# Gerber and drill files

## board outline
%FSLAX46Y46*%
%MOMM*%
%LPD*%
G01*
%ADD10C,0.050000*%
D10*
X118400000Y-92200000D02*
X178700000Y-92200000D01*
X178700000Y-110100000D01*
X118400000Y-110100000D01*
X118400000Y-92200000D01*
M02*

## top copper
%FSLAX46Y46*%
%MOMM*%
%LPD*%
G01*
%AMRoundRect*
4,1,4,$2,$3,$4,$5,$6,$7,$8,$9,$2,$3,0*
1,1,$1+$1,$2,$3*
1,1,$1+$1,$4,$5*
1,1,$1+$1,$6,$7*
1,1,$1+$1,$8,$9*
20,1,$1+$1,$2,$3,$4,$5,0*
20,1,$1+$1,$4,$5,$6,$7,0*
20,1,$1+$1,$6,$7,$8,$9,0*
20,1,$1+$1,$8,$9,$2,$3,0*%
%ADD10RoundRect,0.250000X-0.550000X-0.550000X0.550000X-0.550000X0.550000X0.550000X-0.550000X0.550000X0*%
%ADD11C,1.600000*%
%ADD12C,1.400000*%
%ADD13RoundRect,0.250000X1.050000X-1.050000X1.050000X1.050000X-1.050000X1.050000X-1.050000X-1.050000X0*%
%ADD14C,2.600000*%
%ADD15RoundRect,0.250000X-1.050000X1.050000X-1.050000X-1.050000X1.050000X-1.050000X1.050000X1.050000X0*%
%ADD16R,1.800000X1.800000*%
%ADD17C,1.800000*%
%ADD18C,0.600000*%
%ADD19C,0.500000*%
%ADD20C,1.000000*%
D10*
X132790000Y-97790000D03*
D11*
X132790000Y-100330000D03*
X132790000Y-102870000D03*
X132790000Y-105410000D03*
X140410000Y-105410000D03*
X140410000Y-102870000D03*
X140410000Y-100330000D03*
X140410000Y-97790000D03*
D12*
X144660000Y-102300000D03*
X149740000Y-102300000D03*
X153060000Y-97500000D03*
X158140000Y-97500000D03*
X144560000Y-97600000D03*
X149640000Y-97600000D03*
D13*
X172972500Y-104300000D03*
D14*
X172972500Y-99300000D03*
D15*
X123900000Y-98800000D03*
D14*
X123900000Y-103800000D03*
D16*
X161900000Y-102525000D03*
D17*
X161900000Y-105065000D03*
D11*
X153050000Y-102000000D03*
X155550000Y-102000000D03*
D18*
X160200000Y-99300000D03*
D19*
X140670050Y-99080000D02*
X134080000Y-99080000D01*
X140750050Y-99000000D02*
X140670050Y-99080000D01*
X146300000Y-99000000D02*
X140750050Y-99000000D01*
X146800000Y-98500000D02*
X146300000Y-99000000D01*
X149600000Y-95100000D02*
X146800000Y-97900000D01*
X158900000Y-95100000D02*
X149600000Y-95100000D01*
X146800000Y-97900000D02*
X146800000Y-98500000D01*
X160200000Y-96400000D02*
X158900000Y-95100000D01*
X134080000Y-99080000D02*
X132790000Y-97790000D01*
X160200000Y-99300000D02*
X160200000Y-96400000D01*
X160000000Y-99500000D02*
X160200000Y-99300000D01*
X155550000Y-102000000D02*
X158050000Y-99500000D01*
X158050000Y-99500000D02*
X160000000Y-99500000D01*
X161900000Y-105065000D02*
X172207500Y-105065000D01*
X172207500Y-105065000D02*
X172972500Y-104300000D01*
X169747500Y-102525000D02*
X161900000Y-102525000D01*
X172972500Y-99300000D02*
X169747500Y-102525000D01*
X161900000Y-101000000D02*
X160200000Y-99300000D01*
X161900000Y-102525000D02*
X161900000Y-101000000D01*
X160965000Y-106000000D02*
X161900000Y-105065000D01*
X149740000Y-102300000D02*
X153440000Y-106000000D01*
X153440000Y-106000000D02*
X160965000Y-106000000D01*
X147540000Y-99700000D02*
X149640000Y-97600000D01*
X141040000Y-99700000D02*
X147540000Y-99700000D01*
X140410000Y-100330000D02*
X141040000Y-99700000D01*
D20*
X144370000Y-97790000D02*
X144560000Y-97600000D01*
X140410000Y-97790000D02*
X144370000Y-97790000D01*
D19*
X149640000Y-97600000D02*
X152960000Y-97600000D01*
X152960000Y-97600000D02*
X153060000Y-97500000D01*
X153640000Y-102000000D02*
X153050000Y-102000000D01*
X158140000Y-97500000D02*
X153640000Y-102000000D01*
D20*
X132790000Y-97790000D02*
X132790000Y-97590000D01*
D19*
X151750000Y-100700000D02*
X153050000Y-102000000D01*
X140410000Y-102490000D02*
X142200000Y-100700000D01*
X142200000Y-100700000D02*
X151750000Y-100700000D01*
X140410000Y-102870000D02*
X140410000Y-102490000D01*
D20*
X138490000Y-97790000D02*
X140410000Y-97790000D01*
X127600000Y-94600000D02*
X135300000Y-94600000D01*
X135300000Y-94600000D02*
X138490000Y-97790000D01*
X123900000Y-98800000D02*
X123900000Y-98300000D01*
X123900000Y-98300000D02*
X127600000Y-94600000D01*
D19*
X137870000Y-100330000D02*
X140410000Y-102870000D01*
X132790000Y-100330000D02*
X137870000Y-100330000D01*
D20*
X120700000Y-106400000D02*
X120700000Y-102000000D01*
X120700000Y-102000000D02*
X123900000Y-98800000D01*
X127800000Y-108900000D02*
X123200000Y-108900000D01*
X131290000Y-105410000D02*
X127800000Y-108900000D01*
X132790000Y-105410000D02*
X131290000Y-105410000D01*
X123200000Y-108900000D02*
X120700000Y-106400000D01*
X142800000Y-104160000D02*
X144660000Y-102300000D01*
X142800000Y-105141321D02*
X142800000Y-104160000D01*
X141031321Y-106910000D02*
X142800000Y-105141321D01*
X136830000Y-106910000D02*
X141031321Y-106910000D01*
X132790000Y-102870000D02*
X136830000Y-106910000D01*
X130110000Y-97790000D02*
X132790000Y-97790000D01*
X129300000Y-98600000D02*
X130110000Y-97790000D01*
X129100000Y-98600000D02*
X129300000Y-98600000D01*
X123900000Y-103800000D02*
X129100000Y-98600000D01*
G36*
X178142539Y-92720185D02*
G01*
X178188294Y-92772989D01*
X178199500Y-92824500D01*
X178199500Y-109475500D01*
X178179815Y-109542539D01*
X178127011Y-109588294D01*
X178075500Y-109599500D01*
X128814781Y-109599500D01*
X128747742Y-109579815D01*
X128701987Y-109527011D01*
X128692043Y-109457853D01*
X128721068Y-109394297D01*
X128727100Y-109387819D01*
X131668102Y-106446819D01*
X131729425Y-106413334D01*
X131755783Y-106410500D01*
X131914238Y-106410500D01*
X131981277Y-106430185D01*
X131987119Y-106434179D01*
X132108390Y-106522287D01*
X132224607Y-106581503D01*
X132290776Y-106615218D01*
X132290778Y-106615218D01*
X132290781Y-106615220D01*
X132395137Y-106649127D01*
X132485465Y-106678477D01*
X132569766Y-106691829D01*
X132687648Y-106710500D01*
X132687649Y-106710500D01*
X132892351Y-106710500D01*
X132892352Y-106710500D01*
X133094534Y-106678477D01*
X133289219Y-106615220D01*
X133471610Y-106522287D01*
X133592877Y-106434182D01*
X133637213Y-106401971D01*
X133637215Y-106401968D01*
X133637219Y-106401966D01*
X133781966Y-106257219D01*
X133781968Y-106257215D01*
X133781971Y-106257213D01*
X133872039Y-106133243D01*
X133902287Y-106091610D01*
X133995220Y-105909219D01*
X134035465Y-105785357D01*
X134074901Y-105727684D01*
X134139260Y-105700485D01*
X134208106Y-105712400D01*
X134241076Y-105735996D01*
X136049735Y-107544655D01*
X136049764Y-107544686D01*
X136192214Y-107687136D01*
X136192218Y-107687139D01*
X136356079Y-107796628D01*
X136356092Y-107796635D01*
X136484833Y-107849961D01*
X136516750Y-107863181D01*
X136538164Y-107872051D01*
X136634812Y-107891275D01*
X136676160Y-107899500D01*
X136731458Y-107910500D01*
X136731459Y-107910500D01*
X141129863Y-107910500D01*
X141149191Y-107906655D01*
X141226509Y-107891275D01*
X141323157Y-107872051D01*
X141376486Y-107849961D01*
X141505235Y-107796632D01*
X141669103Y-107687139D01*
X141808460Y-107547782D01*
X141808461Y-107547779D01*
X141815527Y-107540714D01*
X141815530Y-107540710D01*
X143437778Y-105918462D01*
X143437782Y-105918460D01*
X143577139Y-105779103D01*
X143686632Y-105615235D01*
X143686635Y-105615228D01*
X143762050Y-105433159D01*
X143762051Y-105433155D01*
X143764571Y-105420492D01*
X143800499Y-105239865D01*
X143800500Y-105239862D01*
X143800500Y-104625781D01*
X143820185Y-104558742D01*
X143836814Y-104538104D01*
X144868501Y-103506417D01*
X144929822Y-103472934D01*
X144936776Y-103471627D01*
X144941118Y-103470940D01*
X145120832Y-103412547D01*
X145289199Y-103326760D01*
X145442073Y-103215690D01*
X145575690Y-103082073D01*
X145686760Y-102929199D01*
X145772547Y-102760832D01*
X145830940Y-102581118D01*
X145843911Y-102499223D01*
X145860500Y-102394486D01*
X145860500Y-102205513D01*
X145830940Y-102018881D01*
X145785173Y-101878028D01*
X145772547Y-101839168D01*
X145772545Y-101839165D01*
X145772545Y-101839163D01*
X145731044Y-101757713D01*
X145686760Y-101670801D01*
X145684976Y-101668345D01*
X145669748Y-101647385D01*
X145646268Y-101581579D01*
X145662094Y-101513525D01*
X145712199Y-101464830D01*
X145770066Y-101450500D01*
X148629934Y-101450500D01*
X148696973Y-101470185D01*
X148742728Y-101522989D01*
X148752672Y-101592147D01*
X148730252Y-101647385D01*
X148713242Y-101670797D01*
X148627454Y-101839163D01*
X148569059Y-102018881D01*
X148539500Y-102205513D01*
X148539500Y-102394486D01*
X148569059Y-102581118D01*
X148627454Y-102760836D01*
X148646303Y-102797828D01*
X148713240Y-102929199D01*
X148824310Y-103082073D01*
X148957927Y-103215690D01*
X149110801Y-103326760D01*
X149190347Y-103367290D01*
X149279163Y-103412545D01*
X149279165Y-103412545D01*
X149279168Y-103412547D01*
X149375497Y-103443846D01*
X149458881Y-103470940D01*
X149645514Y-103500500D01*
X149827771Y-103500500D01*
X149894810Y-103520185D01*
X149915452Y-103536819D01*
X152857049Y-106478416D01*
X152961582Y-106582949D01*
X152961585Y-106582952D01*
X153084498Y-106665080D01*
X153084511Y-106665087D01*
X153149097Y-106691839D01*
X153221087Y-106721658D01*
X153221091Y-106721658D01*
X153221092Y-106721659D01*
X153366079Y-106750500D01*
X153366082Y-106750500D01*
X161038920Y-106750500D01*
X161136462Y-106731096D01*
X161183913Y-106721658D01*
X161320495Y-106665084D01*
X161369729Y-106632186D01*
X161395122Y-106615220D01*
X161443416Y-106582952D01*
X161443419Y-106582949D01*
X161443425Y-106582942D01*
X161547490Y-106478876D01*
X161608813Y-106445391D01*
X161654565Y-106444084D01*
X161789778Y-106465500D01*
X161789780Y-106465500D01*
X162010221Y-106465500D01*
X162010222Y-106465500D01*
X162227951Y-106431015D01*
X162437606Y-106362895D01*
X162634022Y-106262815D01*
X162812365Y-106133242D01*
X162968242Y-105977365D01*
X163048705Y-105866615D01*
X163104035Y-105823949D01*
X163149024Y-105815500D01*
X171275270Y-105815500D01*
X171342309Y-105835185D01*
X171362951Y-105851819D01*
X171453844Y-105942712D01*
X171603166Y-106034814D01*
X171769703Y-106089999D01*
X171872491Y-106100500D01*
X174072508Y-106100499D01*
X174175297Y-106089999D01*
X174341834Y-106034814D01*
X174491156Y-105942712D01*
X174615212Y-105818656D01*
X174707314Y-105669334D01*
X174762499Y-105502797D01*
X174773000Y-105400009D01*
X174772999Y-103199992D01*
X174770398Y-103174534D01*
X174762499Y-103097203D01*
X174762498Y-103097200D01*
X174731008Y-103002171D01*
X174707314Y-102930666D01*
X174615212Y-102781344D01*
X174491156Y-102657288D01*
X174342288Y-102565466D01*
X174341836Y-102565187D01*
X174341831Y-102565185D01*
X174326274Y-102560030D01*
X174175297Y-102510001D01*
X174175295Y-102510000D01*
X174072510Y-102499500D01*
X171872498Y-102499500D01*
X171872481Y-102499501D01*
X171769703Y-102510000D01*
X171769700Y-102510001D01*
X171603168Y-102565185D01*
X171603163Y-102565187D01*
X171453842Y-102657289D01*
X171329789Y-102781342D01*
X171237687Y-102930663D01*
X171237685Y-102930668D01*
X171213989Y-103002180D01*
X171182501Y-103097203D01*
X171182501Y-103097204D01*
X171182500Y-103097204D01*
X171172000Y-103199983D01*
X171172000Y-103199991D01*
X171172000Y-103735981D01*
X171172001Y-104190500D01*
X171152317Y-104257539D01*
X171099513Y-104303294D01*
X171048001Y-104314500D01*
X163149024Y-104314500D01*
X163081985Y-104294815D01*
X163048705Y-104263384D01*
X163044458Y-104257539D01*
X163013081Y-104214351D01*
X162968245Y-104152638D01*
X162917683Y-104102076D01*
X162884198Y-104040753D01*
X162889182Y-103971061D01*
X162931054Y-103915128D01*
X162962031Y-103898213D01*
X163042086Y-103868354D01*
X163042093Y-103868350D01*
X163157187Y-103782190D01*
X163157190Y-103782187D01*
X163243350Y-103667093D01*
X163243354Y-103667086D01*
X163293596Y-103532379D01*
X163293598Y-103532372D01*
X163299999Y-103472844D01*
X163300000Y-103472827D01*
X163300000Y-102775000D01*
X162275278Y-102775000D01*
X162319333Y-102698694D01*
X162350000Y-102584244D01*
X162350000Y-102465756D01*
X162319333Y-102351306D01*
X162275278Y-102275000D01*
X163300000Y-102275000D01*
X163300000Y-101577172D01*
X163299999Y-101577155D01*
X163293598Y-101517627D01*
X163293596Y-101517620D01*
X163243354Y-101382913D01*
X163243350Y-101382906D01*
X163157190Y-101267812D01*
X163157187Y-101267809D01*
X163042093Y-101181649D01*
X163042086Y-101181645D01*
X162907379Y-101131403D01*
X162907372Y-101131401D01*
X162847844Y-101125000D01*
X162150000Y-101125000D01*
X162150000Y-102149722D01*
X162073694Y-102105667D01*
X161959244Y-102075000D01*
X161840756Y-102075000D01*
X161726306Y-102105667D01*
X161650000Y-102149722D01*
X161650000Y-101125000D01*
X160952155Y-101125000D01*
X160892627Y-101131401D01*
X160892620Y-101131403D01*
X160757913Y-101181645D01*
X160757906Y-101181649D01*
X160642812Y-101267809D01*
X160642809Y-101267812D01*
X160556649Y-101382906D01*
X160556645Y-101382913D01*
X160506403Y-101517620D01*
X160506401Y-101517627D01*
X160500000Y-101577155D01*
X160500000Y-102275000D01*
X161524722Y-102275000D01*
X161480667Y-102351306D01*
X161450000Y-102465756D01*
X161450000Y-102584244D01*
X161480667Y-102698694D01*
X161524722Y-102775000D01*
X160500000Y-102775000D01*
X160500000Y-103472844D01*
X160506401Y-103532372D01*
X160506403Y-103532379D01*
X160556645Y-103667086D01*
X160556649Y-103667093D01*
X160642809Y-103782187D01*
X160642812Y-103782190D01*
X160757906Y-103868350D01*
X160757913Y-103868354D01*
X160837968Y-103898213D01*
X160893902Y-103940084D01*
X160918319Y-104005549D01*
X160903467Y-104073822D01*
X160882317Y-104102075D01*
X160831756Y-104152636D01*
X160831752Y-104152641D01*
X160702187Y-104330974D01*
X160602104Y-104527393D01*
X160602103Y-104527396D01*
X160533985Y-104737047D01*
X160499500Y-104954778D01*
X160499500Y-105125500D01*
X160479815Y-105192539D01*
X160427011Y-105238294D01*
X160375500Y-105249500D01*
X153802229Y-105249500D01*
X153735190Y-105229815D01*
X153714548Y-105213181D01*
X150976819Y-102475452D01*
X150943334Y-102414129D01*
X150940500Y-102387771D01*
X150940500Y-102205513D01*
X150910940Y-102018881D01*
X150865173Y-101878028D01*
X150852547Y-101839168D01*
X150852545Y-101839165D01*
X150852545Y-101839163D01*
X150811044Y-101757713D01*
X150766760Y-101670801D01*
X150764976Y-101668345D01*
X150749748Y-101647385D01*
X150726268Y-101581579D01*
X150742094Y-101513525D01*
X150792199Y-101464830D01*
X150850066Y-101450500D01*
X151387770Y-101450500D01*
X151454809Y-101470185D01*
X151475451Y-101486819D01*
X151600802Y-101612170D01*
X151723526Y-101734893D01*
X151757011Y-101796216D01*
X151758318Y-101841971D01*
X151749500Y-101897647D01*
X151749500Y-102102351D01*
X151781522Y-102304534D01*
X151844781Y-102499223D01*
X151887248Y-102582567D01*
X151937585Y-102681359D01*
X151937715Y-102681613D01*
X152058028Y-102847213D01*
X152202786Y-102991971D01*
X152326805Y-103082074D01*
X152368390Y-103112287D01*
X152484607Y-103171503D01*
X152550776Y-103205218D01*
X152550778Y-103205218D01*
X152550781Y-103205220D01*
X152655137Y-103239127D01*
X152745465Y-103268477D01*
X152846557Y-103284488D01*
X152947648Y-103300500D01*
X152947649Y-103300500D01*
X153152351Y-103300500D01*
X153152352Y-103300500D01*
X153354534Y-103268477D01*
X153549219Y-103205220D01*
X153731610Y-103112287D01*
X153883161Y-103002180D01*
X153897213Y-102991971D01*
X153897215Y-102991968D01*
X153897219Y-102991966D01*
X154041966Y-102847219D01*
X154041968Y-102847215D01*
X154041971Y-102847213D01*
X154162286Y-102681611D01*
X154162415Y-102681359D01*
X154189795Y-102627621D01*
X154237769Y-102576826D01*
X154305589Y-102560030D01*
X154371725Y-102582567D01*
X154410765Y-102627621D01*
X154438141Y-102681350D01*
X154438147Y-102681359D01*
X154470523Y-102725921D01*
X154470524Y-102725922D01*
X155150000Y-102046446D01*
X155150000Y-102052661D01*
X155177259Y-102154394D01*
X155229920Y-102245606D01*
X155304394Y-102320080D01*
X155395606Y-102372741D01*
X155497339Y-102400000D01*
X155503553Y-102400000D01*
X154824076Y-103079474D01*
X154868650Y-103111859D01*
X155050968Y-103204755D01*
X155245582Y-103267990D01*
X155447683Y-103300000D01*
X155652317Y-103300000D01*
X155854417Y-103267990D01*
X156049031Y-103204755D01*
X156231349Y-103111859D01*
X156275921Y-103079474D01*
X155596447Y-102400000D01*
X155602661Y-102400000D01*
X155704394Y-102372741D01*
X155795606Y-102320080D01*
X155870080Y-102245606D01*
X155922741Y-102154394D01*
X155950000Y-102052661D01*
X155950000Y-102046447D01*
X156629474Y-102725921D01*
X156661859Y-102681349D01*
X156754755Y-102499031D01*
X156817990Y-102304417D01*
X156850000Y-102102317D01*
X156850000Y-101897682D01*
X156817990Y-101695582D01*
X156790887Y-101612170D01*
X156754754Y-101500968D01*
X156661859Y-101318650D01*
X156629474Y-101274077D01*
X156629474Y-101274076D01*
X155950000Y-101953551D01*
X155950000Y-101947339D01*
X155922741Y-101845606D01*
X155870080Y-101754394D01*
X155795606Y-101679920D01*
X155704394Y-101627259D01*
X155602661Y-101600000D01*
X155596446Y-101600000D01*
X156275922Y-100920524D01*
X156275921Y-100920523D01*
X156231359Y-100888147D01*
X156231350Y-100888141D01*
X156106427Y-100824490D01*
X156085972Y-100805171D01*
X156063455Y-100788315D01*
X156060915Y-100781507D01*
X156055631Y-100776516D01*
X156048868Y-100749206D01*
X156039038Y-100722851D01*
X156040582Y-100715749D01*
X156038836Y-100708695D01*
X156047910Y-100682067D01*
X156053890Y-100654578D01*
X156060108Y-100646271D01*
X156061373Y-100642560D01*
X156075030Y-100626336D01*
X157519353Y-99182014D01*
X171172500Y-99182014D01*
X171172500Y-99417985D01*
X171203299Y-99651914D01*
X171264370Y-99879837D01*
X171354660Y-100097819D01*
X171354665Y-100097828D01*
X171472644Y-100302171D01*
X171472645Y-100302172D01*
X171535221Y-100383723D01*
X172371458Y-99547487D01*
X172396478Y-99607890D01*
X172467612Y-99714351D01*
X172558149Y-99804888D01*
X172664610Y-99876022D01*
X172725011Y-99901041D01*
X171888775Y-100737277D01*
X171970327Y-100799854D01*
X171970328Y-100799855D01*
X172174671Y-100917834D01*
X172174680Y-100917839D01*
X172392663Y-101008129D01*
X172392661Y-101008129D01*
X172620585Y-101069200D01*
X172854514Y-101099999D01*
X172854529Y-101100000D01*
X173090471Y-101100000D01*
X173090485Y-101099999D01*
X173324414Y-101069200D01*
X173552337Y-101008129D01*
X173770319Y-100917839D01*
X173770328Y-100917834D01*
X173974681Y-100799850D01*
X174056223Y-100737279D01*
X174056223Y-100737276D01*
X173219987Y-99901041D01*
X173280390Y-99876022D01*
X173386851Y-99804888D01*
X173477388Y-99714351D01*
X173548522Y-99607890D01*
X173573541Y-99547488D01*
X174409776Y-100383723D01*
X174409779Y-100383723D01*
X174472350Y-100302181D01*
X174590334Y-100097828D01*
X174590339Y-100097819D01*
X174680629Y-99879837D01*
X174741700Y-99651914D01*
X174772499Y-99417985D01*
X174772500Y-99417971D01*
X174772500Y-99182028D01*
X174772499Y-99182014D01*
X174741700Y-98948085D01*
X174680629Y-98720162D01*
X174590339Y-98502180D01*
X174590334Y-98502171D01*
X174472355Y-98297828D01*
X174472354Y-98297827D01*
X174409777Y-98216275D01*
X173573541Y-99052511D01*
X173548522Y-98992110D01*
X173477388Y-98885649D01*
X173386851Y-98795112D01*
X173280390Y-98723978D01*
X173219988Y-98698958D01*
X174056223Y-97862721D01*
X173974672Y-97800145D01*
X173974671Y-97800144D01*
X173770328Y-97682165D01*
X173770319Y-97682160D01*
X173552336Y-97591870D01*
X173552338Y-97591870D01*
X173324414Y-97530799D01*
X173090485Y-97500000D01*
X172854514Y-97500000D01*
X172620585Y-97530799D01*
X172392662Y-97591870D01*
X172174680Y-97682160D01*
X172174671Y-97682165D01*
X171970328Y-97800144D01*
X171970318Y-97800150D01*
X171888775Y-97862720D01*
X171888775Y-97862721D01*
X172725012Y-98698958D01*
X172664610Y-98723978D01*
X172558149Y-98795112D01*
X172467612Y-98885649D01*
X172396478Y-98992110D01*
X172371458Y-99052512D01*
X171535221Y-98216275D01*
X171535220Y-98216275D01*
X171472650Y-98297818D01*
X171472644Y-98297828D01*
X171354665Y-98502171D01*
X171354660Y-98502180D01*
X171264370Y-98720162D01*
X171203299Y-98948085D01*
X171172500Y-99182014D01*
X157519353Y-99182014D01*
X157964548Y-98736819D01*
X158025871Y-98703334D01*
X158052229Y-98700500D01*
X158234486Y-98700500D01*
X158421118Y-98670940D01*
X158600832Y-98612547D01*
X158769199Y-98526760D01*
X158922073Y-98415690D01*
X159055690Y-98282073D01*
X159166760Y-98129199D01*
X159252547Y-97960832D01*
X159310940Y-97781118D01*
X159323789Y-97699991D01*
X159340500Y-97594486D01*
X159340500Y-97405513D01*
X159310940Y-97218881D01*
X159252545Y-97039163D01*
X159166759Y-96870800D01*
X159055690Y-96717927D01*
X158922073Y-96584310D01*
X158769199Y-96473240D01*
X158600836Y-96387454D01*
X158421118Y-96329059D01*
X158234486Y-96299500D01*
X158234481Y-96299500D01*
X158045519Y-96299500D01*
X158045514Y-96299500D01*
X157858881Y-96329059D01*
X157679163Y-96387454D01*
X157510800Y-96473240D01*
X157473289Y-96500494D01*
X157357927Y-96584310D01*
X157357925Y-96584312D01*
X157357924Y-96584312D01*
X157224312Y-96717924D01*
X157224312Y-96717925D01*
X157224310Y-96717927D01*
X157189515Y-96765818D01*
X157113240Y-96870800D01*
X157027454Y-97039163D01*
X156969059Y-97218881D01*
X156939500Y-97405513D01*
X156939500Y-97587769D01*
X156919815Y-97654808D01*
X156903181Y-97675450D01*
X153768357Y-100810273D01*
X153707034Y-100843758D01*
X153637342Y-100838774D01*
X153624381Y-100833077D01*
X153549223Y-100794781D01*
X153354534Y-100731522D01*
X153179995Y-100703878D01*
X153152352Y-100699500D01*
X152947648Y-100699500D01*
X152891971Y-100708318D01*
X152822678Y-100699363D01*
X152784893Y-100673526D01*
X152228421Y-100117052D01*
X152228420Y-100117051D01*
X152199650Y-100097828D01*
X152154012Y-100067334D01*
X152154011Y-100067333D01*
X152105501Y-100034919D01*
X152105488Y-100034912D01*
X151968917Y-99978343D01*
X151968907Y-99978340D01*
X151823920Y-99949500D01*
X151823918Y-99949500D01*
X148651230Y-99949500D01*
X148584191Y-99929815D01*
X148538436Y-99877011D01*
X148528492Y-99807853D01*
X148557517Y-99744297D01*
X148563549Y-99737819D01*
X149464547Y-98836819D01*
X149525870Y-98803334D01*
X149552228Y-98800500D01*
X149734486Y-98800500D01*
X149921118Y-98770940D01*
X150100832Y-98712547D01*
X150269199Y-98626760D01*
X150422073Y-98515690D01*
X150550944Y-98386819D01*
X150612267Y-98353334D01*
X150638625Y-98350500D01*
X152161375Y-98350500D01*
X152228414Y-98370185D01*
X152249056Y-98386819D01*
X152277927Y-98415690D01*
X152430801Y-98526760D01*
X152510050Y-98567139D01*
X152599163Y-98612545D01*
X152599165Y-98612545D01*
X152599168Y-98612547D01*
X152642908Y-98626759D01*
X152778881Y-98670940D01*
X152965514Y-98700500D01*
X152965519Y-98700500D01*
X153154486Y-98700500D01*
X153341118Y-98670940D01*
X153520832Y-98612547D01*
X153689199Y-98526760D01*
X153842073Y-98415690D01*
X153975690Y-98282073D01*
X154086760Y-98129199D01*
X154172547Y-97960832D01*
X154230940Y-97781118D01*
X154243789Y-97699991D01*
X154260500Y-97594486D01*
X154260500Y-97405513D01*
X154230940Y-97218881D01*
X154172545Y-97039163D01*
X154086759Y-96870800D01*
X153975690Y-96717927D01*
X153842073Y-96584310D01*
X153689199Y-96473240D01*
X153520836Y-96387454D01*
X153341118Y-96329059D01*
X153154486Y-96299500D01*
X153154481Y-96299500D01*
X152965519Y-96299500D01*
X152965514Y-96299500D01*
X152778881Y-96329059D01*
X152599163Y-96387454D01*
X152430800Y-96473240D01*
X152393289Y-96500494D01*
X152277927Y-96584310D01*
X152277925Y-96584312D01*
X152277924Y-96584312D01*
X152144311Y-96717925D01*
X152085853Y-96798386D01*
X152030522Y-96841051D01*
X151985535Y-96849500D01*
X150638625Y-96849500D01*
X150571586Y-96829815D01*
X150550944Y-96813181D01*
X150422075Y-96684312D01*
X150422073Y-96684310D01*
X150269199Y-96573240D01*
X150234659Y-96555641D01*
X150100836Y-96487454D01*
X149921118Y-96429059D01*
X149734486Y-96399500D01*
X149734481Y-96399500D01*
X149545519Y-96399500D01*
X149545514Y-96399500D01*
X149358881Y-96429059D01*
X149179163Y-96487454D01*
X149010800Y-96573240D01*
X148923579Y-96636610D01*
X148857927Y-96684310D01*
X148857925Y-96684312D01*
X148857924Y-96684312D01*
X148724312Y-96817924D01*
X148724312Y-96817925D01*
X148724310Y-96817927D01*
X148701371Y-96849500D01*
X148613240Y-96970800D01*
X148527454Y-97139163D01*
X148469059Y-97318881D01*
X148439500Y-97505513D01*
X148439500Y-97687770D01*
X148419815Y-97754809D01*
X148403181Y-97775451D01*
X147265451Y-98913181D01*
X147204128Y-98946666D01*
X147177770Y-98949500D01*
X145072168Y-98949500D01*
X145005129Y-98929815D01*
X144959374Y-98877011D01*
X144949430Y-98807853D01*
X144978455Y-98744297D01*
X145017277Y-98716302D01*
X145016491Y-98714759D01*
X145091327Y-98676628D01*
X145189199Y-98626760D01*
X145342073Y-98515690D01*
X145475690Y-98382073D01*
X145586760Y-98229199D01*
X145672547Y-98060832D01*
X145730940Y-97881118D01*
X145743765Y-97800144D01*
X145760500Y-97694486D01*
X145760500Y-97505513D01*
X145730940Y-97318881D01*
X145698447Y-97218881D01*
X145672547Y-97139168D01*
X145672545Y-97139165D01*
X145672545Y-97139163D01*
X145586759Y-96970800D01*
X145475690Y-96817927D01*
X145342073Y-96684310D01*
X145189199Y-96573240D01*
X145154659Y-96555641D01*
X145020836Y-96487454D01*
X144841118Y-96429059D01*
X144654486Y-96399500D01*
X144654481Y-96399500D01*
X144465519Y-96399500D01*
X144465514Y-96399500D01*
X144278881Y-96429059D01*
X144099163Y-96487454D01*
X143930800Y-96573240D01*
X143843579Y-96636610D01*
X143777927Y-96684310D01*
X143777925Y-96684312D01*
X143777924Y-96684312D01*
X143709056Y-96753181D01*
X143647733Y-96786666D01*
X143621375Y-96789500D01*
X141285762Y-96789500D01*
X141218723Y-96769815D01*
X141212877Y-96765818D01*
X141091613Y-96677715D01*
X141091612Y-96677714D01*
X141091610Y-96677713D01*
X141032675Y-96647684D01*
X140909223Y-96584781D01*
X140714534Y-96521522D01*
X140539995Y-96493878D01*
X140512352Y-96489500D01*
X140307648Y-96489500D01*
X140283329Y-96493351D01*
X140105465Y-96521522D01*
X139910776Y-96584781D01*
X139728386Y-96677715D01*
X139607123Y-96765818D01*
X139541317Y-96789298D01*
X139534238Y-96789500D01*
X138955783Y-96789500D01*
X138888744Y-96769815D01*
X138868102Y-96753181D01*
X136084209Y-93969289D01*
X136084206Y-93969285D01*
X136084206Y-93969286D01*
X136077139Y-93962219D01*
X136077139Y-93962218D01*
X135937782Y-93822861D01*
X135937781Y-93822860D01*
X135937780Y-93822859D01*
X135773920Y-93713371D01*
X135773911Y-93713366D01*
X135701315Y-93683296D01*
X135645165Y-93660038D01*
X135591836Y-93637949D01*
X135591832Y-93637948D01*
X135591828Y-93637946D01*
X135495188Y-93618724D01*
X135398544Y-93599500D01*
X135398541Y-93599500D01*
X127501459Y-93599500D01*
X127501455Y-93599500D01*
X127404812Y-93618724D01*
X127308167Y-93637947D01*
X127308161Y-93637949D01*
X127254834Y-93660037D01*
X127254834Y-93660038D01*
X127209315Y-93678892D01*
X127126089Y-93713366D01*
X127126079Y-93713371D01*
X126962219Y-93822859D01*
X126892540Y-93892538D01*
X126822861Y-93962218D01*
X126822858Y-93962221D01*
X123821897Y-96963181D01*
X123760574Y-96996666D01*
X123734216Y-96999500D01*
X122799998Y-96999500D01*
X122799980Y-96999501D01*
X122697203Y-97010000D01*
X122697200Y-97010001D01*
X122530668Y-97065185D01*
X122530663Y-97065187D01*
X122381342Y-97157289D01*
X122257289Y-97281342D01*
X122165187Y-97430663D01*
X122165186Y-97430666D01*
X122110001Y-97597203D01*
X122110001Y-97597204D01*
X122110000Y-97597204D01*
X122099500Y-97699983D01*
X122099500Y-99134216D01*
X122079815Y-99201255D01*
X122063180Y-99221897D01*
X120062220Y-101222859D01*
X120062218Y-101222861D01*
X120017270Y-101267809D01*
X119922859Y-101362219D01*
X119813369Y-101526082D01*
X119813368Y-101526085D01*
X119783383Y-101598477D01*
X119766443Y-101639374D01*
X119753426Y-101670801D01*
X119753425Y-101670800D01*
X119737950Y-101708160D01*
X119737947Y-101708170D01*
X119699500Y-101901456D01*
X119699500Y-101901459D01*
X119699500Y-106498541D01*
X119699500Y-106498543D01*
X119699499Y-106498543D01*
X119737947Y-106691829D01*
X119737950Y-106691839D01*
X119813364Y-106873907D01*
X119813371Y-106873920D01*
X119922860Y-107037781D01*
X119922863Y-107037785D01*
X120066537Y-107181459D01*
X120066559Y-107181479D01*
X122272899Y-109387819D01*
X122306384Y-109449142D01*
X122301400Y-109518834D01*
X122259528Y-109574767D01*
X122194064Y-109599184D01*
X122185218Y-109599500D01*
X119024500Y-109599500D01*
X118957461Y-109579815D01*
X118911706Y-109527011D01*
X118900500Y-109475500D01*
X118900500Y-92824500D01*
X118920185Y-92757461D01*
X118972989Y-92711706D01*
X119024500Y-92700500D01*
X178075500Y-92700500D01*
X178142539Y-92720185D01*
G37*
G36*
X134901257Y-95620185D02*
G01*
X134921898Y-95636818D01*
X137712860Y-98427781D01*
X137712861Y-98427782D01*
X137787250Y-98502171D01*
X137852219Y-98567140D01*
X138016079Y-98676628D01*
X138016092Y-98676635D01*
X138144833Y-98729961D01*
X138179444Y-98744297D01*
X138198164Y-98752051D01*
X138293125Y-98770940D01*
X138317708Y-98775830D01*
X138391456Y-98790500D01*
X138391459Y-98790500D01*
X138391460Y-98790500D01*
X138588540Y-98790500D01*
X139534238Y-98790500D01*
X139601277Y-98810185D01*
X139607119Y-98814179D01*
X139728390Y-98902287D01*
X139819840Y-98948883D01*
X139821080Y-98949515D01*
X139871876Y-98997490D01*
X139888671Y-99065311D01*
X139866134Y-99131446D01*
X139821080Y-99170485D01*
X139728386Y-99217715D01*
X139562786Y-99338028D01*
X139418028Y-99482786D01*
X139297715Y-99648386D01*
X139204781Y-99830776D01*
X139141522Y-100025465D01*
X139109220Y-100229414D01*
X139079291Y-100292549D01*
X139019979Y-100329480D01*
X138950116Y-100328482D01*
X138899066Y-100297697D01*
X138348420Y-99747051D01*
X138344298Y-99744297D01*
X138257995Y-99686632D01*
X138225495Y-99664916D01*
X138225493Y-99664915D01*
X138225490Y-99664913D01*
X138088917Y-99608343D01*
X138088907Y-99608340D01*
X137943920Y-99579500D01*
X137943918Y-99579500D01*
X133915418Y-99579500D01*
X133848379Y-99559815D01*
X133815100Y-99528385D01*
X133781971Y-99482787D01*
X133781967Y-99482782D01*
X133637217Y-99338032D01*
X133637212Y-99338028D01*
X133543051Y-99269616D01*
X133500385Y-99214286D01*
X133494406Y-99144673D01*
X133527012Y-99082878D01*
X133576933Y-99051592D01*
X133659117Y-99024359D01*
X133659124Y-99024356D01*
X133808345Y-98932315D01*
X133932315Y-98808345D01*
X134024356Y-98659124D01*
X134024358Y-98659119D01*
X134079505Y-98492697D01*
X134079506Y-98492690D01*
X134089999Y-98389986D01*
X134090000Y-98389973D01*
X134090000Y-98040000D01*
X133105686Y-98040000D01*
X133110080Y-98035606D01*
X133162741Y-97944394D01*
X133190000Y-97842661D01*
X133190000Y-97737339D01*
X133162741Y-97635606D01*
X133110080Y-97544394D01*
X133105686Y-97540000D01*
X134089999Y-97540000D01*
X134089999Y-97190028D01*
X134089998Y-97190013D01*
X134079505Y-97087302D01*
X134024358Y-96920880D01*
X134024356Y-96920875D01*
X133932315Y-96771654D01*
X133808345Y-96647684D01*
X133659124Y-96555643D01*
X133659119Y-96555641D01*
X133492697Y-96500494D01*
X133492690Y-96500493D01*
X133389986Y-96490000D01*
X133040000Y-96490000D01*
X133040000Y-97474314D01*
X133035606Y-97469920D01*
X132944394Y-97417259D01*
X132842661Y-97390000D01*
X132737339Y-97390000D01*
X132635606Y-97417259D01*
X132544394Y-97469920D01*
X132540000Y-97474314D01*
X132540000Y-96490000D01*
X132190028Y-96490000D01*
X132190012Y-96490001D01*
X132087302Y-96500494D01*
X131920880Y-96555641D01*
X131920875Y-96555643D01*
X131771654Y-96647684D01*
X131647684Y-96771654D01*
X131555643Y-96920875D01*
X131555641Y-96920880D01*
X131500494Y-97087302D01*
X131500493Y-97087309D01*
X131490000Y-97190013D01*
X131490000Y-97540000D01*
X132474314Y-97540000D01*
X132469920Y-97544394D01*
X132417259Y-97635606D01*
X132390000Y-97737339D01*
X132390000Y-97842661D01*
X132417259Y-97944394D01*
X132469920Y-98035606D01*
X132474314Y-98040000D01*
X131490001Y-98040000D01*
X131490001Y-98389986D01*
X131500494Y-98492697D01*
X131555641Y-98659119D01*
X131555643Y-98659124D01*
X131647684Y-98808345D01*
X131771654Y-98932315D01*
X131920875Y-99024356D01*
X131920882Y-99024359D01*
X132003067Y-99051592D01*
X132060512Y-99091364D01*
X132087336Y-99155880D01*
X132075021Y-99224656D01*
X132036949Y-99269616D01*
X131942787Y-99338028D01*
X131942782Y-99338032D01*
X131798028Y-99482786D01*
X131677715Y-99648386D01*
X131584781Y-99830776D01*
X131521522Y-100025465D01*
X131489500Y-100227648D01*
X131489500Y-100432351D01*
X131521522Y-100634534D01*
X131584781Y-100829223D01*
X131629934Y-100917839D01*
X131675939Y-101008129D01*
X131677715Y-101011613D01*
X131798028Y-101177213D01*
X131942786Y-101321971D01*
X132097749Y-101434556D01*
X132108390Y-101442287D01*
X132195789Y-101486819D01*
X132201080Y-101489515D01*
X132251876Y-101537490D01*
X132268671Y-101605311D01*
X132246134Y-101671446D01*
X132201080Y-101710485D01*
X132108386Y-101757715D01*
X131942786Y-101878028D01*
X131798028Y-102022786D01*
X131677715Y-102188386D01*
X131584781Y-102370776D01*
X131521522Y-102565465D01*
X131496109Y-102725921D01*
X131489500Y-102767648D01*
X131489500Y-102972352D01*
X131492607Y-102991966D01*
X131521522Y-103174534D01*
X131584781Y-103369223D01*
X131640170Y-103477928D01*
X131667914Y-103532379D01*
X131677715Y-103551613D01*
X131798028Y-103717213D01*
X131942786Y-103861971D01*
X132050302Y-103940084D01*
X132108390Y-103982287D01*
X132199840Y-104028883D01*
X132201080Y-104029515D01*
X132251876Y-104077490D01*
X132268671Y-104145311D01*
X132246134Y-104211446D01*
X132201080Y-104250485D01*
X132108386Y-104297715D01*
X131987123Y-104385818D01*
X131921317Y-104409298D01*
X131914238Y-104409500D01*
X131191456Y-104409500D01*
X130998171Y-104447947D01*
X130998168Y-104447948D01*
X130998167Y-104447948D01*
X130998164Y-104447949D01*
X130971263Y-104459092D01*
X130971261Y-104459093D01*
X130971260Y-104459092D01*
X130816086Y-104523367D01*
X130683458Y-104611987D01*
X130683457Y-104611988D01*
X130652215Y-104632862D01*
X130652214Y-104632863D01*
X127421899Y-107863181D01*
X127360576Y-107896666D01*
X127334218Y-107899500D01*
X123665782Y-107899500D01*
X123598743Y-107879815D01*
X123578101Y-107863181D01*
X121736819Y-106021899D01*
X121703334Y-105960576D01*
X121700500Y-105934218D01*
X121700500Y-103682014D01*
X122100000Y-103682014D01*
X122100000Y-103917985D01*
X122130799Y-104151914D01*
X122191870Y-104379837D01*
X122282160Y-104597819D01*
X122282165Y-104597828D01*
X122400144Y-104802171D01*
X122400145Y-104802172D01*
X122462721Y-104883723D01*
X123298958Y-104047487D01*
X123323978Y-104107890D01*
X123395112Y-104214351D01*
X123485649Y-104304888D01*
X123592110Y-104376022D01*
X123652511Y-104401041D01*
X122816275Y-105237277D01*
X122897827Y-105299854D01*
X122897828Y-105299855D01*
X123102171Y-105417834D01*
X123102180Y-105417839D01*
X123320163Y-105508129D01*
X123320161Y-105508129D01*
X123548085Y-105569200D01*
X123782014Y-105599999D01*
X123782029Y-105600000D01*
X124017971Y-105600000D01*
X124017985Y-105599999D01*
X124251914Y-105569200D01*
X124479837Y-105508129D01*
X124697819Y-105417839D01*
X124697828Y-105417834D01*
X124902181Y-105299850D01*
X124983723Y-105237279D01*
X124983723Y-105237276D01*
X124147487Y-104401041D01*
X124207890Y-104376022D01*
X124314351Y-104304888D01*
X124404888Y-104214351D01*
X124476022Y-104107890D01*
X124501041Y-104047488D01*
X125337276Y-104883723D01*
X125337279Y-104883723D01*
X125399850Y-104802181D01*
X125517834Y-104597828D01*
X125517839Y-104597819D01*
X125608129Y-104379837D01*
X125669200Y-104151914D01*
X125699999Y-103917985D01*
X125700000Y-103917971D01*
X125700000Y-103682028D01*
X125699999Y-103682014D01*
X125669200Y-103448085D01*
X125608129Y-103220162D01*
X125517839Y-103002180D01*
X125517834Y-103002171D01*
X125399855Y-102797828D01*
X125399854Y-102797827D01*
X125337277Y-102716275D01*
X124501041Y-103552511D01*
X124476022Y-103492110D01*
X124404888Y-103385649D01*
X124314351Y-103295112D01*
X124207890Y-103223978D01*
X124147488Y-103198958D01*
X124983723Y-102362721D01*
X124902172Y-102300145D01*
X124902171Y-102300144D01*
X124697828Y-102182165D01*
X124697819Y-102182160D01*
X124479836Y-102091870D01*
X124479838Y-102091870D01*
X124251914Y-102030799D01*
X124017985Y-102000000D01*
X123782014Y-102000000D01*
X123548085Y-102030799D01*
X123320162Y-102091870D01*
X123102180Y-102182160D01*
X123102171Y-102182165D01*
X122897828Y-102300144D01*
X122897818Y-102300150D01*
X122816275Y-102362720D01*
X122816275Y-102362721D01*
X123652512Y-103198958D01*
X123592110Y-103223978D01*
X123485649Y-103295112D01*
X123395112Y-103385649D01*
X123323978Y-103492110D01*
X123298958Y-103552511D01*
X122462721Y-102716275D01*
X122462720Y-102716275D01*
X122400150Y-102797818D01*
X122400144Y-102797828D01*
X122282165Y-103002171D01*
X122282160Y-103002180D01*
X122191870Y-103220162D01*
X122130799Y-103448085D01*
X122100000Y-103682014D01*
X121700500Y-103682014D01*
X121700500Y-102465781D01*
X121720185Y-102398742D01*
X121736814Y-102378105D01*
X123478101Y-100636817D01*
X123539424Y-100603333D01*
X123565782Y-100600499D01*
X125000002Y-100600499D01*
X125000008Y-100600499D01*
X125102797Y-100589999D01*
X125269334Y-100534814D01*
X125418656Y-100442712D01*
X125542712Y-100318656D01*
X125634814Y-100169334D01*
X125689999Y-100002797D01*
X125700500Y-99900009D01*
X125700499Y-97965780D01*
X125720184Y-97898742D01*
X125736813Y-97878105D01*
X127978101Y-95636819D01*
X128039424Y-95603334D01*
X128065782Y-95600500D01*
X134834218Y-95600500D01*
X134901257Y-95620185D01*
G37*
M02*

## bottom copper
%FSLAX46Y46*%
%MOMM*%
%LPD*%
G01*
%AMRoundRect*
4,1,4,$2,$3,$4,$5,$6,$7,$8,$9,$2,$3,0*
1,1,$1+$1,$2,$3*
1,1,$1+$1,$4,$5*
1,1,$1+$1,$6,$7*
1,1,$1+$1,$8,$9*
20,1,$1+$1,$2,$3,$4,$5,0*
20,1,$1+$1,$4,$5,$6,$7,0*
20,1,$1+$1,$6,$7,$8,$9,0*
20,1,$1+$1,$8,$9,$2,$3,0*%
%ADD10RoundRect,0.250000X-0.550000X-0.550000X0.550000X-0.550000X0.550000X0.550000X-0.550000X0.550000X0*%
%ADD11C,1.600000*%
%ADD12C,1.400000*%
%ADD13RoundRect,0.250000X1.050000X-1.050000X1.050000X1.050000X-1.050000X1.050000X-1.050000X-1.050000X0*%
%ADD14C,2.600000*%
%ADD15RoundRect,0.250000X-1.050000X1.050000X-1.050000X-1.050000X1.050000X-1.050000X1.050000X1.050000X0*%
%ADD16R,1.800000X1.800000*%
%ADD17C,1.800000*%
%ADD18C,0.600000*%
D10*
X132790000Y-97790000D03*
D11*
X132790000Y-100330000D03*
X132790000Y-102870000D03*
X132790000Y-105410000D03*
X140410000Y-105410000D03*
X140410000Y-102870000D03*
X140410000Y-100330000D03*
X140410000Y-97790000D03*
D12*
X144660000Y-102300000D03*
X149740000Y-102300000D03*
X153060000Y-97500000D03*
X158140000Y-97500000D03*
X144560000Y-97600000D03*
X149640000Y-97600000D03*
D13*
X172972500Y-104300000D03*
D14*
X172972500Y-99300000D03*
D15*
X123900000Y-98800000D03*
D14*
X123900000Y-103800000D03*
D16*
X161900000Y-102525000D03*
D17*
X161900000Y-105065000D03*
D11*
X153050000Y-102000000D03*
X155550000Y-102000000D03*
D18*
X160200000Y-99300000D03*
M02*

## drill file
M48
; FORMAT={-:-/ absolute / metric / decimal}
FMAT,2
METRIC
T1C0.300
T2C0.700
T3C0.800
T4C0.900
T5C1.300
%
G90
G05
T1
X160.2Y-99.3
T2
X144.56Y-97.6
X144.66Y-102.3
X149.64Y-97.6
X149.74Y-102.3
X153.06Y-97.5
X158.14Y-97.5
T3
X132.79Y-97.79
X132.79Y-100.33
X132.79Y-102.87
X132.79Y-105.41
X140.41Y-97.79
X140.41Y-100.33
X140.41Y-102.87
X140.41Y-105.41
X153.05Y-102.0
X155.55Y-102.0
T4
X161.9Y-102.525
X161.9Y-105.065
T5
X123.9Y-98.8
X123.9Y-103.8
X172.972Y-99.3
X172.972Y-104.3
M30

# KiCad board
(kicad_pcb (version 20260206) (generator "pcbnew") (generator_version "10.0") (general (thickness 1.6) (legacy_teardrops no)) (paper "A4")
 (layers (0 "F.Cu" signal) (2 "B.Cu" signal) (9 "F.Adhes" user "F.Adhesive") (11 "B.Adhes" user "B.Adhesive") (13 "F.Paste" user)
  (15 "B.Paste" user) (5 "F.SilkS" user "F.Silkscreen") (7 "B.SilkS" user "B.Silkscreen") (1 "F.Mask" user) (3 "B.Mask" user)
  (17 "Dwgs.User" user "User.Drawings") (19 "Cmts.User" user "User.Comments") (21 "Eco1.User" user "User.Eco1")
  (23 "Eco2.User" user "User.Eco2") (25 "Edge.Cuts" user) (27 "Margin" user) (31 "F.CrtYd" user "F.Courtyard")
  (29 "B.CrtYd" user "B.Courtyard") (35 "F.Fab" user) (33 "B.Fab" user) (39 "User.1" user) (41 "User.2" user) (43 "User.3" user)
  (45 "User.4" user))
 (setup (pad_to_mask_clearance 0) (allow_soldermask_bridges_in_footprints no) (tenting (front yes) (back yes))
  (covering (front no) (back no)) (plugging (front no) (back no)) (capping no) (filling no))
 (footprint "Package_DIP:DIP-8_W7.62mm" (layer "F.Cu") (at 132.79 97.79)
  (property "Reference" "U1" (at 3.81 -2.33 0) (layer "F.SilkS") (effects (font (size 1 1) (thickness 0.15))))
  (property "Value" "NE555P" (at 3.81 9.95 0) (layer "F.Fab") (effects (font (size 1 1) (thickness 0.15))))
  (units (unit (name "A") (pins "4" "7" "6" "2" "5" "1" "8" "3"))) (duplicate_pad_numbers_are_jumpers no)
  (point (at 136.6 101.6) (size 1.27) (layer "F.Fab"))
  (pad "1" thru_hole roundrect (at 0 0) (size 1.6 1.6) (drill 0.8) (layers "*.Cu" "*.Mask") (remove_unused_layers no)
   (roundrect_rratio 0.15625) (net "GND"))
  (pad "2" thru_hole circle (at 0 2.54) (size 1.6 1.6) (drill 0.8) (layers "*.Cu" "*.Mask") (remove_unused_layers no) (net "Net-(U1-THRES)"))
  (pad "3" thru_hole circle (at 0 5.08) (size 1.6 1.6) (drill 0.8) (layers "*.Cu" "*.Mask") (remove_unused_layers no) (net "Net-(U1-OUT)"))
  (pad "4" thru_hole circle (at 0 7.62) (size 1.6 1.6) (drill 0.8) (layers "*.Cu" "*.Mask") (remove_unused_layers no) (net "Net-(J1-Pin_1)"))
  (pad "5" thru_hole circle (at 7.62 7.62) (size 1.6 1.6) (drill 0.8) (layers "*.Cu" "*.Mask") (remove_unused_layers no)
   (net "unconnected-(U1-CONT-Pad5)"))
  (pad "6" thru_hole circle (at 7.62 5.08) (size 1.6 1.6) (drill 0.8) (layers "*.Cu" "*.Mask") (remove_unused_layers no)
   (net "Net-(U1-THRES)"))
  (pad "7" thru_hole circle (at 7.62 2.54) (size 1.6 1.6) (drill 0.8) (layers "*.Cu" "*.Mask") (remove_unused_layers no)
   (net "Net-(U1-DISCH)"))
  (pad "8" thru_hole circle (at 7.62 0) (size 1.6 1.6) (drill 0.8) (layers "*.Cu" "*.Mask") (remove_unused_layers no) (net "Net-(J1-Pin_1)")))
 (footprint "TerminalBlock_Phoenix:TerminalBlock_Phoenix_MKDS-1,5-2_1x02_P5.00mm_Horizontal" (layer "F.Cu") (at 172.9725 104.3 90)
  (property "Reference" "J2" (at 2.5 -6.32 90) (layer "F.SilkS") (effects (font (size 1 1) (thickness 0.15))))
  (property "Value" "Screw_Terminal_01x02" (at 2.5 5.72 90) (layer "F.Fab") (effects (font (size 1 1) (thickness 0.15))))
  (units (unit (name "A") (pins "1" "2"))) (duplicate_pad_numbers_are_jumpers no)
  (pad "1" thru_hole roundrect (at 0 0 90) (size 2.6 2.6) (drill 1.3) (layers "*.Cu" "*.Mask") (remove_unused_layers no)
   (roundrect_rratio 0.096154) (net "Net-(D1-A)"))
  (pad "2" thru_hole circle (at 5 0 90) (size 2.6 2.6) (drill 1.3) (layers "*.Cu" "*.Mask") (remove_unused_layers no) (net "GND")))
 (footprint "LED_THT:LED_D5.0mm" (layer "F.Cu") (at 161.9 102.525 -90)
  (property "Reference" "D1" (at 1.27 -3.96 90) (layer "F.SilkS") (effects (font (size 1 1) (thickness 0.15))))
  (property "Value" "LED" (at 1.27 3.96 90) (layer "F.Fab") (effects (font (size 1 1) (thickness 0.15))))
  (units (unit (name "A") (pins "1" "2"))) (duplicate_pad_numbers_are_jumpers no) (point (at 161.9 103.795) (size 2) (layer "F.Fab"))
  (pad "1" thru_hole rect (at 0 0 270) (size 1.8 1.8) (drill 0.9) (layers "*.Cu" "*.Mask") (remove_unused_layers no) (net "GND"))
  (pad "2" thru_hole circle (at 2.54 0 270) (size 1.8 1.8) (drill 0.9) (layers "*.Cu" "*.Mask") (remove_unused_layers no) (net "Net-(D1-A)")))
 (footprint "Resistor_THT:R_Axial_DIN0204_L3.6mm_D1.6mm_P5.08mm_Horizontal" (layer "F.Cu") (at 153.06 97.5)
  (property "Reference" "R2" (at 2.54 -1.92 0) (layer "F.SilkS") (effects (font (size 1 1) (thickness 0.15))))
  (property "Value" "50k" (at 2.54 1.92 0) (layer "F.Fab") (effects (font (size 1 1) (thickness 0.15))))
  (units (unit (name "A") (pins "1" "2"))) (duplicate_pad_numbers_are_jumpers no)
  (pad "1" thru_hole circle (at 0 0) (size 1.4 1.4) (drill 0.7) (layers "*.Cu" "*.Mask") (remove_unused_layers no) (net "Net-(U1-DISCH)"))
  (pad "2" thru_hole circle (at 5.08 0) (size 1.4 1.4) (drill 0.7) (layers "*.Cu" "*.Mask") (remove_unused_layers no) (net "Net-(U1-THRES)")))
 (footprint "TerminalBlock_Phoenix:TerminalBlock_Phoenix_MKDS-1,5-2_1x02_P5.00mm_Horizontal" (layer "F.Cu") (at 123.9 98.8 -90)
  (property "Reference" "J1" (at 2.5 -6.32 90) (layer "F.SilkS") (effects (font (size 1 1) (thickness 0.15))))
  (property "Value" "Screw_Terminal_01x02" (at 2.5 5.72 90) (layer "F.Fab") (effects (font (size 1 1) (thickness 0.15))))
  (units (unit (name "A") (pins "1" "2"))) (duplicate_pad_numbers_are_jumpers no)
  (pad "1" thru_hole roundrect (at 0 0 270) (size 2.6 2.6) (drill 1.3) (layers "*.Cu" "*.Mask") (remove_unused_layers no)
   (roundrect_rratio 0.096154) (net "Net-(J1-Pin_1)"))
  (pad "2" thru_hole circle (at 5 0 270) (size 2.6 2.6) (drill 1.3) (layers "*.Cu" "*.Mask") (remove_unused_layers no) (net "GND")))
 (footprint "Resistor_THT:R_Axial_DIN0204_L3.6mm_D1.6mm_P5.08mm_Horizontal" (layer "F.Cu") (at 144.56 97.6)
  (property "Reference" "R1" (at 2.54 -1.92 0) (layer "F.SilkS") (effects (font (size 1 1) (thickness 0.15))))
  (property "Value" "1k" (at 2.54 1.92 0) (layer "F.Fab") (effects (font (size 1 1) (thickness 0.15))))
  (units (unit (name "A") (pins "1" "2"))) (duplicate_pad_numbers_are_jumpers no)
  (pad "1" thru_hole circle (at 0 0) (size 1.4 1.4) (drill 0.7) (layers "*.Cu" "*.Mask") (remove_unused_layers no) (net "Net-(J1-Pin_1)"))
  (pad "2" thru_hole circle (at 5.08 0) (size 1.4 1.4) (drill 0.7) (layers "*.Cu" "*.Mask") (remove_unused_layers no) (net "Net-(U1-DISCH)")))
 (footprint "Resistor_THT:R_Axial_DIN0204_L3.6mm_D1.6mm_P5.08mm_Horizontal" (layer "F.Cu") (at 144.66 102.3)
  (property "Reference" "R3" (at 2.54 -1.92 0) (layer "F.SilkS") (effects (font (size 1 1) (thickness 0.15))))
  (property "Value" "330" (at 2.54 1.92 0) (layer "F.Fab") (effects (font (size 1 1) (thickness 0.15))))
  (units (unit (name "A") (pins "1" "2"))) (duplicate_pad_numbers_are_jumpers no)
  (pad "1" thru_hole circle (at 0 0) (size 1.4 1.4) (drill 0.7) (layers "*.Cu" "*.Mask") (remove_unused_layers no) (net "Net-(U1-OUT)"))
  (pad "2" thru_hole circle (at 5.08 0) (size 1.4 1.4) (drill 0.7) (layers "*.Cu" "*.Mask") (remove_unused_layers no) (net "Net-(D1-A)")))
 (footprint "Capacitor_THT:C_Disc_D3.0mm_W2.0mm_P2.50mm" (layer "F.Cu") (at 153.05 102)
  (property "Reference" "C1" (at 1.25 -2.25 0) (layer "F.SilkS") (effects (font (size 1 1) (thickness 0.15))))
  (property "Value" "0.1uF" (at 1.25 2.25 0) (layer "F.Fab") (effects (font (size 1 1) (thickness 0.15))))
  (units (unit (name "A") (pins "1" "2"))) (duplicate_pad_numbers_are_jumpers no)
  (pad "1" thru_hole circle (at 0 0) (size 1.6 1.6) (drill 0.8) (layers "*.Cu" "*.Mask") (remove_unused_layers no) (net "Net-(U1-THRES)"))
  (pad "2" thru_hole circle (at 2.5 0) (size 1.6 1.6) (drill 0.8) (layers "*.Cu" "*.Mask") (remove_unused_layers no) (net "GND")))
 (gr_rect (start 118.4 92.2) (end 178.7 110.1) (stroke (width 0.05) (type default)) (fill no) (layer "Edge.Cuts"))
 (segment (start 129.1 98.6) (end 129.3 98.6) (width 1) (layer "F.Cu") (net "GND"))
 (segment (start 158.9 95.1) (end 149.6 95.1) (width 0.5) (layer "F.Cu") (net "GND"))
 (segment (start 132.79 97.79) (end 132.79 97.59) (width 1) (layer "F.Cu") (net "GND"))
 (segment (start 149.6 95.1) (end 146.8 97.9) (width 0.5) (layer "F.Cu") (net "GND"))
 (segment (start 123.9 103.8) (end 129.1 98.6) (width 1) (layer "F.Cu") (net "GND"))
 (segment (start 158.05 99.5) (end 160 99.5) (width 0.5) (layer "F.Cu") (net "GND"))
 (segment (start 146.8 98.5) (end 146.3 99) (width 0.5) (layer "F.Cu") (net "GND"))
 (segment (start 155.55 102) (end 158.05 99.5) (width 0.5) (layer "F.Cu") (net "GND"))
 (segment (start 129.3 98.6) (end 130.11 97.79) (width 1) (layer "F.Cu") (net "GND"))
 (segment (start 130.11 97.79) (end 132.79 97.79) (width 1) (layer "F.Cu") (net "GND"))
 (segment (start 160.2 99.3) (end 160.2 96.4) (width 0.5) (layer "F.Cu") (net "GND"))
 (segment (start 146.3 99) (end 140.75005 99) (width 0.5) (layer "F.Cu") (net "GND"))
 (segment (start 140.75005 99) (end 140.67005 99.08) (width 0.5) (layer "F.Cu") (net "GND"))
 (segment (start 161.9 102.525) (end 161.9 101) (width 0.5) (layer "F.Cu") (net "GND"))
 (segment (start 160.2 96.4) (end 158.9 95.1) (width 0.5) (layer "F.Cu") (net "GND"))
 (segment (start 172.9725 99.3) (end 169.7475 102.525) (width 0.5) (layer "F.Cu") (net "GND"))
 (segment (start 169.7475 102.525) (end 161.9 102.525) (width 0.5) (layer "F.Cu") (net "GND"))
 (segment (start 161.9 101) (end 160.2 99.3) (width 0.5) (layer "F.Cu") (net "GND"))
 (segment (start 160 99.5) (end 160.2 99.3) (width 0.5) (layer "F.Cu") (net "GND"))
 (segment (start 146.8 97.9) (end 146.8 98.5) (width 0.5) (layer "F.Cu") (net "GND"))
 (segment (start 140.67005 99.08) (end 134.08 99.08) (width 0.5) (layer "F.Cu") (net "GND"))
 (segment (start 134.08 99.08) (end 132.79 97.79) (width 0.5) (layer "F.Cu") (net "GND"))
 (via (at 160.2 99.3) (size 0.6) (drill 0.3) (layers "F.Cu" "B.Cu") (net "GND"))
 (segment (start 140.41 102.87) (end 140.41 102.49) (width 0.5) (layer "F.Cu") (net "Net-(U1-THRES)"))
 (segment (start 140.41 102.49) (end 142.2 100.7) (width 0.5) (layer "F.Cu") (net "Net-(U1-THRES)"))
 (segment (start 153.64 102) (end 153.05 102) (width 0.5) (layer "F.Cu") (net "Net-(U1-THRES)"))
 (segment (start 137.87 100.33) (end 140.41 102.87) (width 0.5) (layer "F.Cu") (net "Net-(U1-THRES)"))
 (segment (start 132.79 100.33) (end 137.87 100.33) (width 0.5) (layer "F.Cu") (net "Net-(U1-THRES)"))
 (segment (start 142.2 100.7) (end 151.75 100.7) (width 0.5) (layer "F.Cu") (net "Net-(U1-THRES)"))
 (segment (start 151.75 100.7) (end 153.05 102) (width 0.5) (layer "F.Cu") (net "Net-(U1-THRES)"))
 (segment (start 158.14 97.5) (end 153.64 102) (width 0.5) (layer "F.Cu") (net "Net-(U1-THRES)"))
 (segment (start 153.44 106) (end 160.965 106) (width 0.5) (layer "F.Cu") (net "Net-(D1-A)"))
 (segment (start 172.2075 105.065) (end 172.9725 104.3) (width 0.5) (layer "F.Cu") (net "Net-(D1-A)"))
 (segment (start 149.74 102.3) (end 153.44 106) (width 0.5) (layer "F.Cu") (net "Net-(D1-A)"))
 (segment (start 160.965 106) (end 161.9 105.065) (width 0.5) (layer "F.Cu") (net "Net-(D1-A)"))
 (segment (start 161.9 105.065) (end 172.2075 105.065) (width 0.5) (layer "F.Cu") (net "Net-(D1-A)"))
 (segment (start 144.37 97.79) (end 144.56 97.6) (width 1) (layer "F.Cu") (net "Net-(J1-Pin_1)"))
 (segment (start 123.9 98.8) (end 123.9 98.3) (width 1) (layer "F.Cu") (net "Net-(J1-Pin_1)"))
 (segment (start 132.79 105.41) (end 131.29 105.41) (width 1) (layer "F.Cu") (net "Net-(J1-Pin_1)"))
 (segment (start 120.7 106.4) (end 120.7 102) (width 1) (layer "F.Cu") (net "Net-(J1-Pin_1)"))
 (segment (start 127.6 94.6) (end 135.3 94.6) (width 1) (layer "F.Cu") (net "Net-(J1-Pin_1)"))
 (segment (start 123.2 108.9) (end 120.7 106.4) (width 1) (layer "F.Cu") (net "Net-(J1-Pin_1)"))
 (segment (start 138.49 97.79) (end 140.41 97.79) (width 1) (layer "F.Cu") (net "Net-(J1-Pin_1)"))
 (segment (start 127.8 108.9) (end 123.2 108.9) (width 1) (layer "F.Cu") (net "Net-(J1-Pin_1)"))
 (segment (start 120.7 102) (end 123.9 98.8) (width 1) (layer "F.Cu") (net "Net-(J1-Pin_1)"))
 (segment (start 123.9 98.3) (end 127.6 94.6) (width 1) (layer "F.Cu") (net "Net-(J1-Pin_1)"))
 (segment (start 140.41 97.79) (end 144.37 97.79) (width 1) (layer "F.Cu") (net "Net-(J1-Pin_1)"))
 (segment (start 131.29 105.41) (end 127.8 108.9) (width 1) (layer "F.Cu") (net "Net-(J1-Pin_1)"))
 (segment (start 135.3 94.6) (end 138.49 97.79) (width 1) (layer "F.Cu") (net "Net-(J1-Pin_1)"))
 (segment (start 152.96 97.6) (end 153.06 97.5) (width 0.5) (layer "F.Cu") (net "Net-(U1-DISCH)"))
 (segment (start 140.41 100.33) (end 141.04 99.7) (width 0.5) (layer "F.Cu") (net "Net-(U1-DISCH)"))
 (segment (start 141.04 99.7) (end 147.54 99.7) (width 0.5) (layer "F.Cu") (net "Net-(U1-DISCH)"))
 (segment (start 149.64 97.6) (end 152.96 97.6) (width 0.5) (layer "F.Cu") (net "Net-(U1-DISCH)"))
 (segment (start 147.54 99.7) (end 149.64 97.6) (width 0.5) (layer "F.Cu") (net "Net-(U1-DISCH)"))
 (segment (start 141.031321 106.91) (end 142.8 105.141321) (width 1) (layer "F.Cu") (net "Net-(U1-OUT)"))
 (segment (start 132.79 102.87) (end 136.83 106.91) (width 1) (layer "F.Cu") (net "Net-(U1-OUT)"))
 (segment (start 142.8 105.141321) (end 142.8 104.16) (width 1) (layer "F.Cu") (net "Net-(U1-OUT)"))
 (segment (start 142.8 104.16) (end 144.66 102.3) (width 1) (layer "F.Cu") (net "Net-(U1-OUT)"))
 (segment (start 136.83 106.91) (end 141.031321 106.91) (width 1) (layer "F.Cu") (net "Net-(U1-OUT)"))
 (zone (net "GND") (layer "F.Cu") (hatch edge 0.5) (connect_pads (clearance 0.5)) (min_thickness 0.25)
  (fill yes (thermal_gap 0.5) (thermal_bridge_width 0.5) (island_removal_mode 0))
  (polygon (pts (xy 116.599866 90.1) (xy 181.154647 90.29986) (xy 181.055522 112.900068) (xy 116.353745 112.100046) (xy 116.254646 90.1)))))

